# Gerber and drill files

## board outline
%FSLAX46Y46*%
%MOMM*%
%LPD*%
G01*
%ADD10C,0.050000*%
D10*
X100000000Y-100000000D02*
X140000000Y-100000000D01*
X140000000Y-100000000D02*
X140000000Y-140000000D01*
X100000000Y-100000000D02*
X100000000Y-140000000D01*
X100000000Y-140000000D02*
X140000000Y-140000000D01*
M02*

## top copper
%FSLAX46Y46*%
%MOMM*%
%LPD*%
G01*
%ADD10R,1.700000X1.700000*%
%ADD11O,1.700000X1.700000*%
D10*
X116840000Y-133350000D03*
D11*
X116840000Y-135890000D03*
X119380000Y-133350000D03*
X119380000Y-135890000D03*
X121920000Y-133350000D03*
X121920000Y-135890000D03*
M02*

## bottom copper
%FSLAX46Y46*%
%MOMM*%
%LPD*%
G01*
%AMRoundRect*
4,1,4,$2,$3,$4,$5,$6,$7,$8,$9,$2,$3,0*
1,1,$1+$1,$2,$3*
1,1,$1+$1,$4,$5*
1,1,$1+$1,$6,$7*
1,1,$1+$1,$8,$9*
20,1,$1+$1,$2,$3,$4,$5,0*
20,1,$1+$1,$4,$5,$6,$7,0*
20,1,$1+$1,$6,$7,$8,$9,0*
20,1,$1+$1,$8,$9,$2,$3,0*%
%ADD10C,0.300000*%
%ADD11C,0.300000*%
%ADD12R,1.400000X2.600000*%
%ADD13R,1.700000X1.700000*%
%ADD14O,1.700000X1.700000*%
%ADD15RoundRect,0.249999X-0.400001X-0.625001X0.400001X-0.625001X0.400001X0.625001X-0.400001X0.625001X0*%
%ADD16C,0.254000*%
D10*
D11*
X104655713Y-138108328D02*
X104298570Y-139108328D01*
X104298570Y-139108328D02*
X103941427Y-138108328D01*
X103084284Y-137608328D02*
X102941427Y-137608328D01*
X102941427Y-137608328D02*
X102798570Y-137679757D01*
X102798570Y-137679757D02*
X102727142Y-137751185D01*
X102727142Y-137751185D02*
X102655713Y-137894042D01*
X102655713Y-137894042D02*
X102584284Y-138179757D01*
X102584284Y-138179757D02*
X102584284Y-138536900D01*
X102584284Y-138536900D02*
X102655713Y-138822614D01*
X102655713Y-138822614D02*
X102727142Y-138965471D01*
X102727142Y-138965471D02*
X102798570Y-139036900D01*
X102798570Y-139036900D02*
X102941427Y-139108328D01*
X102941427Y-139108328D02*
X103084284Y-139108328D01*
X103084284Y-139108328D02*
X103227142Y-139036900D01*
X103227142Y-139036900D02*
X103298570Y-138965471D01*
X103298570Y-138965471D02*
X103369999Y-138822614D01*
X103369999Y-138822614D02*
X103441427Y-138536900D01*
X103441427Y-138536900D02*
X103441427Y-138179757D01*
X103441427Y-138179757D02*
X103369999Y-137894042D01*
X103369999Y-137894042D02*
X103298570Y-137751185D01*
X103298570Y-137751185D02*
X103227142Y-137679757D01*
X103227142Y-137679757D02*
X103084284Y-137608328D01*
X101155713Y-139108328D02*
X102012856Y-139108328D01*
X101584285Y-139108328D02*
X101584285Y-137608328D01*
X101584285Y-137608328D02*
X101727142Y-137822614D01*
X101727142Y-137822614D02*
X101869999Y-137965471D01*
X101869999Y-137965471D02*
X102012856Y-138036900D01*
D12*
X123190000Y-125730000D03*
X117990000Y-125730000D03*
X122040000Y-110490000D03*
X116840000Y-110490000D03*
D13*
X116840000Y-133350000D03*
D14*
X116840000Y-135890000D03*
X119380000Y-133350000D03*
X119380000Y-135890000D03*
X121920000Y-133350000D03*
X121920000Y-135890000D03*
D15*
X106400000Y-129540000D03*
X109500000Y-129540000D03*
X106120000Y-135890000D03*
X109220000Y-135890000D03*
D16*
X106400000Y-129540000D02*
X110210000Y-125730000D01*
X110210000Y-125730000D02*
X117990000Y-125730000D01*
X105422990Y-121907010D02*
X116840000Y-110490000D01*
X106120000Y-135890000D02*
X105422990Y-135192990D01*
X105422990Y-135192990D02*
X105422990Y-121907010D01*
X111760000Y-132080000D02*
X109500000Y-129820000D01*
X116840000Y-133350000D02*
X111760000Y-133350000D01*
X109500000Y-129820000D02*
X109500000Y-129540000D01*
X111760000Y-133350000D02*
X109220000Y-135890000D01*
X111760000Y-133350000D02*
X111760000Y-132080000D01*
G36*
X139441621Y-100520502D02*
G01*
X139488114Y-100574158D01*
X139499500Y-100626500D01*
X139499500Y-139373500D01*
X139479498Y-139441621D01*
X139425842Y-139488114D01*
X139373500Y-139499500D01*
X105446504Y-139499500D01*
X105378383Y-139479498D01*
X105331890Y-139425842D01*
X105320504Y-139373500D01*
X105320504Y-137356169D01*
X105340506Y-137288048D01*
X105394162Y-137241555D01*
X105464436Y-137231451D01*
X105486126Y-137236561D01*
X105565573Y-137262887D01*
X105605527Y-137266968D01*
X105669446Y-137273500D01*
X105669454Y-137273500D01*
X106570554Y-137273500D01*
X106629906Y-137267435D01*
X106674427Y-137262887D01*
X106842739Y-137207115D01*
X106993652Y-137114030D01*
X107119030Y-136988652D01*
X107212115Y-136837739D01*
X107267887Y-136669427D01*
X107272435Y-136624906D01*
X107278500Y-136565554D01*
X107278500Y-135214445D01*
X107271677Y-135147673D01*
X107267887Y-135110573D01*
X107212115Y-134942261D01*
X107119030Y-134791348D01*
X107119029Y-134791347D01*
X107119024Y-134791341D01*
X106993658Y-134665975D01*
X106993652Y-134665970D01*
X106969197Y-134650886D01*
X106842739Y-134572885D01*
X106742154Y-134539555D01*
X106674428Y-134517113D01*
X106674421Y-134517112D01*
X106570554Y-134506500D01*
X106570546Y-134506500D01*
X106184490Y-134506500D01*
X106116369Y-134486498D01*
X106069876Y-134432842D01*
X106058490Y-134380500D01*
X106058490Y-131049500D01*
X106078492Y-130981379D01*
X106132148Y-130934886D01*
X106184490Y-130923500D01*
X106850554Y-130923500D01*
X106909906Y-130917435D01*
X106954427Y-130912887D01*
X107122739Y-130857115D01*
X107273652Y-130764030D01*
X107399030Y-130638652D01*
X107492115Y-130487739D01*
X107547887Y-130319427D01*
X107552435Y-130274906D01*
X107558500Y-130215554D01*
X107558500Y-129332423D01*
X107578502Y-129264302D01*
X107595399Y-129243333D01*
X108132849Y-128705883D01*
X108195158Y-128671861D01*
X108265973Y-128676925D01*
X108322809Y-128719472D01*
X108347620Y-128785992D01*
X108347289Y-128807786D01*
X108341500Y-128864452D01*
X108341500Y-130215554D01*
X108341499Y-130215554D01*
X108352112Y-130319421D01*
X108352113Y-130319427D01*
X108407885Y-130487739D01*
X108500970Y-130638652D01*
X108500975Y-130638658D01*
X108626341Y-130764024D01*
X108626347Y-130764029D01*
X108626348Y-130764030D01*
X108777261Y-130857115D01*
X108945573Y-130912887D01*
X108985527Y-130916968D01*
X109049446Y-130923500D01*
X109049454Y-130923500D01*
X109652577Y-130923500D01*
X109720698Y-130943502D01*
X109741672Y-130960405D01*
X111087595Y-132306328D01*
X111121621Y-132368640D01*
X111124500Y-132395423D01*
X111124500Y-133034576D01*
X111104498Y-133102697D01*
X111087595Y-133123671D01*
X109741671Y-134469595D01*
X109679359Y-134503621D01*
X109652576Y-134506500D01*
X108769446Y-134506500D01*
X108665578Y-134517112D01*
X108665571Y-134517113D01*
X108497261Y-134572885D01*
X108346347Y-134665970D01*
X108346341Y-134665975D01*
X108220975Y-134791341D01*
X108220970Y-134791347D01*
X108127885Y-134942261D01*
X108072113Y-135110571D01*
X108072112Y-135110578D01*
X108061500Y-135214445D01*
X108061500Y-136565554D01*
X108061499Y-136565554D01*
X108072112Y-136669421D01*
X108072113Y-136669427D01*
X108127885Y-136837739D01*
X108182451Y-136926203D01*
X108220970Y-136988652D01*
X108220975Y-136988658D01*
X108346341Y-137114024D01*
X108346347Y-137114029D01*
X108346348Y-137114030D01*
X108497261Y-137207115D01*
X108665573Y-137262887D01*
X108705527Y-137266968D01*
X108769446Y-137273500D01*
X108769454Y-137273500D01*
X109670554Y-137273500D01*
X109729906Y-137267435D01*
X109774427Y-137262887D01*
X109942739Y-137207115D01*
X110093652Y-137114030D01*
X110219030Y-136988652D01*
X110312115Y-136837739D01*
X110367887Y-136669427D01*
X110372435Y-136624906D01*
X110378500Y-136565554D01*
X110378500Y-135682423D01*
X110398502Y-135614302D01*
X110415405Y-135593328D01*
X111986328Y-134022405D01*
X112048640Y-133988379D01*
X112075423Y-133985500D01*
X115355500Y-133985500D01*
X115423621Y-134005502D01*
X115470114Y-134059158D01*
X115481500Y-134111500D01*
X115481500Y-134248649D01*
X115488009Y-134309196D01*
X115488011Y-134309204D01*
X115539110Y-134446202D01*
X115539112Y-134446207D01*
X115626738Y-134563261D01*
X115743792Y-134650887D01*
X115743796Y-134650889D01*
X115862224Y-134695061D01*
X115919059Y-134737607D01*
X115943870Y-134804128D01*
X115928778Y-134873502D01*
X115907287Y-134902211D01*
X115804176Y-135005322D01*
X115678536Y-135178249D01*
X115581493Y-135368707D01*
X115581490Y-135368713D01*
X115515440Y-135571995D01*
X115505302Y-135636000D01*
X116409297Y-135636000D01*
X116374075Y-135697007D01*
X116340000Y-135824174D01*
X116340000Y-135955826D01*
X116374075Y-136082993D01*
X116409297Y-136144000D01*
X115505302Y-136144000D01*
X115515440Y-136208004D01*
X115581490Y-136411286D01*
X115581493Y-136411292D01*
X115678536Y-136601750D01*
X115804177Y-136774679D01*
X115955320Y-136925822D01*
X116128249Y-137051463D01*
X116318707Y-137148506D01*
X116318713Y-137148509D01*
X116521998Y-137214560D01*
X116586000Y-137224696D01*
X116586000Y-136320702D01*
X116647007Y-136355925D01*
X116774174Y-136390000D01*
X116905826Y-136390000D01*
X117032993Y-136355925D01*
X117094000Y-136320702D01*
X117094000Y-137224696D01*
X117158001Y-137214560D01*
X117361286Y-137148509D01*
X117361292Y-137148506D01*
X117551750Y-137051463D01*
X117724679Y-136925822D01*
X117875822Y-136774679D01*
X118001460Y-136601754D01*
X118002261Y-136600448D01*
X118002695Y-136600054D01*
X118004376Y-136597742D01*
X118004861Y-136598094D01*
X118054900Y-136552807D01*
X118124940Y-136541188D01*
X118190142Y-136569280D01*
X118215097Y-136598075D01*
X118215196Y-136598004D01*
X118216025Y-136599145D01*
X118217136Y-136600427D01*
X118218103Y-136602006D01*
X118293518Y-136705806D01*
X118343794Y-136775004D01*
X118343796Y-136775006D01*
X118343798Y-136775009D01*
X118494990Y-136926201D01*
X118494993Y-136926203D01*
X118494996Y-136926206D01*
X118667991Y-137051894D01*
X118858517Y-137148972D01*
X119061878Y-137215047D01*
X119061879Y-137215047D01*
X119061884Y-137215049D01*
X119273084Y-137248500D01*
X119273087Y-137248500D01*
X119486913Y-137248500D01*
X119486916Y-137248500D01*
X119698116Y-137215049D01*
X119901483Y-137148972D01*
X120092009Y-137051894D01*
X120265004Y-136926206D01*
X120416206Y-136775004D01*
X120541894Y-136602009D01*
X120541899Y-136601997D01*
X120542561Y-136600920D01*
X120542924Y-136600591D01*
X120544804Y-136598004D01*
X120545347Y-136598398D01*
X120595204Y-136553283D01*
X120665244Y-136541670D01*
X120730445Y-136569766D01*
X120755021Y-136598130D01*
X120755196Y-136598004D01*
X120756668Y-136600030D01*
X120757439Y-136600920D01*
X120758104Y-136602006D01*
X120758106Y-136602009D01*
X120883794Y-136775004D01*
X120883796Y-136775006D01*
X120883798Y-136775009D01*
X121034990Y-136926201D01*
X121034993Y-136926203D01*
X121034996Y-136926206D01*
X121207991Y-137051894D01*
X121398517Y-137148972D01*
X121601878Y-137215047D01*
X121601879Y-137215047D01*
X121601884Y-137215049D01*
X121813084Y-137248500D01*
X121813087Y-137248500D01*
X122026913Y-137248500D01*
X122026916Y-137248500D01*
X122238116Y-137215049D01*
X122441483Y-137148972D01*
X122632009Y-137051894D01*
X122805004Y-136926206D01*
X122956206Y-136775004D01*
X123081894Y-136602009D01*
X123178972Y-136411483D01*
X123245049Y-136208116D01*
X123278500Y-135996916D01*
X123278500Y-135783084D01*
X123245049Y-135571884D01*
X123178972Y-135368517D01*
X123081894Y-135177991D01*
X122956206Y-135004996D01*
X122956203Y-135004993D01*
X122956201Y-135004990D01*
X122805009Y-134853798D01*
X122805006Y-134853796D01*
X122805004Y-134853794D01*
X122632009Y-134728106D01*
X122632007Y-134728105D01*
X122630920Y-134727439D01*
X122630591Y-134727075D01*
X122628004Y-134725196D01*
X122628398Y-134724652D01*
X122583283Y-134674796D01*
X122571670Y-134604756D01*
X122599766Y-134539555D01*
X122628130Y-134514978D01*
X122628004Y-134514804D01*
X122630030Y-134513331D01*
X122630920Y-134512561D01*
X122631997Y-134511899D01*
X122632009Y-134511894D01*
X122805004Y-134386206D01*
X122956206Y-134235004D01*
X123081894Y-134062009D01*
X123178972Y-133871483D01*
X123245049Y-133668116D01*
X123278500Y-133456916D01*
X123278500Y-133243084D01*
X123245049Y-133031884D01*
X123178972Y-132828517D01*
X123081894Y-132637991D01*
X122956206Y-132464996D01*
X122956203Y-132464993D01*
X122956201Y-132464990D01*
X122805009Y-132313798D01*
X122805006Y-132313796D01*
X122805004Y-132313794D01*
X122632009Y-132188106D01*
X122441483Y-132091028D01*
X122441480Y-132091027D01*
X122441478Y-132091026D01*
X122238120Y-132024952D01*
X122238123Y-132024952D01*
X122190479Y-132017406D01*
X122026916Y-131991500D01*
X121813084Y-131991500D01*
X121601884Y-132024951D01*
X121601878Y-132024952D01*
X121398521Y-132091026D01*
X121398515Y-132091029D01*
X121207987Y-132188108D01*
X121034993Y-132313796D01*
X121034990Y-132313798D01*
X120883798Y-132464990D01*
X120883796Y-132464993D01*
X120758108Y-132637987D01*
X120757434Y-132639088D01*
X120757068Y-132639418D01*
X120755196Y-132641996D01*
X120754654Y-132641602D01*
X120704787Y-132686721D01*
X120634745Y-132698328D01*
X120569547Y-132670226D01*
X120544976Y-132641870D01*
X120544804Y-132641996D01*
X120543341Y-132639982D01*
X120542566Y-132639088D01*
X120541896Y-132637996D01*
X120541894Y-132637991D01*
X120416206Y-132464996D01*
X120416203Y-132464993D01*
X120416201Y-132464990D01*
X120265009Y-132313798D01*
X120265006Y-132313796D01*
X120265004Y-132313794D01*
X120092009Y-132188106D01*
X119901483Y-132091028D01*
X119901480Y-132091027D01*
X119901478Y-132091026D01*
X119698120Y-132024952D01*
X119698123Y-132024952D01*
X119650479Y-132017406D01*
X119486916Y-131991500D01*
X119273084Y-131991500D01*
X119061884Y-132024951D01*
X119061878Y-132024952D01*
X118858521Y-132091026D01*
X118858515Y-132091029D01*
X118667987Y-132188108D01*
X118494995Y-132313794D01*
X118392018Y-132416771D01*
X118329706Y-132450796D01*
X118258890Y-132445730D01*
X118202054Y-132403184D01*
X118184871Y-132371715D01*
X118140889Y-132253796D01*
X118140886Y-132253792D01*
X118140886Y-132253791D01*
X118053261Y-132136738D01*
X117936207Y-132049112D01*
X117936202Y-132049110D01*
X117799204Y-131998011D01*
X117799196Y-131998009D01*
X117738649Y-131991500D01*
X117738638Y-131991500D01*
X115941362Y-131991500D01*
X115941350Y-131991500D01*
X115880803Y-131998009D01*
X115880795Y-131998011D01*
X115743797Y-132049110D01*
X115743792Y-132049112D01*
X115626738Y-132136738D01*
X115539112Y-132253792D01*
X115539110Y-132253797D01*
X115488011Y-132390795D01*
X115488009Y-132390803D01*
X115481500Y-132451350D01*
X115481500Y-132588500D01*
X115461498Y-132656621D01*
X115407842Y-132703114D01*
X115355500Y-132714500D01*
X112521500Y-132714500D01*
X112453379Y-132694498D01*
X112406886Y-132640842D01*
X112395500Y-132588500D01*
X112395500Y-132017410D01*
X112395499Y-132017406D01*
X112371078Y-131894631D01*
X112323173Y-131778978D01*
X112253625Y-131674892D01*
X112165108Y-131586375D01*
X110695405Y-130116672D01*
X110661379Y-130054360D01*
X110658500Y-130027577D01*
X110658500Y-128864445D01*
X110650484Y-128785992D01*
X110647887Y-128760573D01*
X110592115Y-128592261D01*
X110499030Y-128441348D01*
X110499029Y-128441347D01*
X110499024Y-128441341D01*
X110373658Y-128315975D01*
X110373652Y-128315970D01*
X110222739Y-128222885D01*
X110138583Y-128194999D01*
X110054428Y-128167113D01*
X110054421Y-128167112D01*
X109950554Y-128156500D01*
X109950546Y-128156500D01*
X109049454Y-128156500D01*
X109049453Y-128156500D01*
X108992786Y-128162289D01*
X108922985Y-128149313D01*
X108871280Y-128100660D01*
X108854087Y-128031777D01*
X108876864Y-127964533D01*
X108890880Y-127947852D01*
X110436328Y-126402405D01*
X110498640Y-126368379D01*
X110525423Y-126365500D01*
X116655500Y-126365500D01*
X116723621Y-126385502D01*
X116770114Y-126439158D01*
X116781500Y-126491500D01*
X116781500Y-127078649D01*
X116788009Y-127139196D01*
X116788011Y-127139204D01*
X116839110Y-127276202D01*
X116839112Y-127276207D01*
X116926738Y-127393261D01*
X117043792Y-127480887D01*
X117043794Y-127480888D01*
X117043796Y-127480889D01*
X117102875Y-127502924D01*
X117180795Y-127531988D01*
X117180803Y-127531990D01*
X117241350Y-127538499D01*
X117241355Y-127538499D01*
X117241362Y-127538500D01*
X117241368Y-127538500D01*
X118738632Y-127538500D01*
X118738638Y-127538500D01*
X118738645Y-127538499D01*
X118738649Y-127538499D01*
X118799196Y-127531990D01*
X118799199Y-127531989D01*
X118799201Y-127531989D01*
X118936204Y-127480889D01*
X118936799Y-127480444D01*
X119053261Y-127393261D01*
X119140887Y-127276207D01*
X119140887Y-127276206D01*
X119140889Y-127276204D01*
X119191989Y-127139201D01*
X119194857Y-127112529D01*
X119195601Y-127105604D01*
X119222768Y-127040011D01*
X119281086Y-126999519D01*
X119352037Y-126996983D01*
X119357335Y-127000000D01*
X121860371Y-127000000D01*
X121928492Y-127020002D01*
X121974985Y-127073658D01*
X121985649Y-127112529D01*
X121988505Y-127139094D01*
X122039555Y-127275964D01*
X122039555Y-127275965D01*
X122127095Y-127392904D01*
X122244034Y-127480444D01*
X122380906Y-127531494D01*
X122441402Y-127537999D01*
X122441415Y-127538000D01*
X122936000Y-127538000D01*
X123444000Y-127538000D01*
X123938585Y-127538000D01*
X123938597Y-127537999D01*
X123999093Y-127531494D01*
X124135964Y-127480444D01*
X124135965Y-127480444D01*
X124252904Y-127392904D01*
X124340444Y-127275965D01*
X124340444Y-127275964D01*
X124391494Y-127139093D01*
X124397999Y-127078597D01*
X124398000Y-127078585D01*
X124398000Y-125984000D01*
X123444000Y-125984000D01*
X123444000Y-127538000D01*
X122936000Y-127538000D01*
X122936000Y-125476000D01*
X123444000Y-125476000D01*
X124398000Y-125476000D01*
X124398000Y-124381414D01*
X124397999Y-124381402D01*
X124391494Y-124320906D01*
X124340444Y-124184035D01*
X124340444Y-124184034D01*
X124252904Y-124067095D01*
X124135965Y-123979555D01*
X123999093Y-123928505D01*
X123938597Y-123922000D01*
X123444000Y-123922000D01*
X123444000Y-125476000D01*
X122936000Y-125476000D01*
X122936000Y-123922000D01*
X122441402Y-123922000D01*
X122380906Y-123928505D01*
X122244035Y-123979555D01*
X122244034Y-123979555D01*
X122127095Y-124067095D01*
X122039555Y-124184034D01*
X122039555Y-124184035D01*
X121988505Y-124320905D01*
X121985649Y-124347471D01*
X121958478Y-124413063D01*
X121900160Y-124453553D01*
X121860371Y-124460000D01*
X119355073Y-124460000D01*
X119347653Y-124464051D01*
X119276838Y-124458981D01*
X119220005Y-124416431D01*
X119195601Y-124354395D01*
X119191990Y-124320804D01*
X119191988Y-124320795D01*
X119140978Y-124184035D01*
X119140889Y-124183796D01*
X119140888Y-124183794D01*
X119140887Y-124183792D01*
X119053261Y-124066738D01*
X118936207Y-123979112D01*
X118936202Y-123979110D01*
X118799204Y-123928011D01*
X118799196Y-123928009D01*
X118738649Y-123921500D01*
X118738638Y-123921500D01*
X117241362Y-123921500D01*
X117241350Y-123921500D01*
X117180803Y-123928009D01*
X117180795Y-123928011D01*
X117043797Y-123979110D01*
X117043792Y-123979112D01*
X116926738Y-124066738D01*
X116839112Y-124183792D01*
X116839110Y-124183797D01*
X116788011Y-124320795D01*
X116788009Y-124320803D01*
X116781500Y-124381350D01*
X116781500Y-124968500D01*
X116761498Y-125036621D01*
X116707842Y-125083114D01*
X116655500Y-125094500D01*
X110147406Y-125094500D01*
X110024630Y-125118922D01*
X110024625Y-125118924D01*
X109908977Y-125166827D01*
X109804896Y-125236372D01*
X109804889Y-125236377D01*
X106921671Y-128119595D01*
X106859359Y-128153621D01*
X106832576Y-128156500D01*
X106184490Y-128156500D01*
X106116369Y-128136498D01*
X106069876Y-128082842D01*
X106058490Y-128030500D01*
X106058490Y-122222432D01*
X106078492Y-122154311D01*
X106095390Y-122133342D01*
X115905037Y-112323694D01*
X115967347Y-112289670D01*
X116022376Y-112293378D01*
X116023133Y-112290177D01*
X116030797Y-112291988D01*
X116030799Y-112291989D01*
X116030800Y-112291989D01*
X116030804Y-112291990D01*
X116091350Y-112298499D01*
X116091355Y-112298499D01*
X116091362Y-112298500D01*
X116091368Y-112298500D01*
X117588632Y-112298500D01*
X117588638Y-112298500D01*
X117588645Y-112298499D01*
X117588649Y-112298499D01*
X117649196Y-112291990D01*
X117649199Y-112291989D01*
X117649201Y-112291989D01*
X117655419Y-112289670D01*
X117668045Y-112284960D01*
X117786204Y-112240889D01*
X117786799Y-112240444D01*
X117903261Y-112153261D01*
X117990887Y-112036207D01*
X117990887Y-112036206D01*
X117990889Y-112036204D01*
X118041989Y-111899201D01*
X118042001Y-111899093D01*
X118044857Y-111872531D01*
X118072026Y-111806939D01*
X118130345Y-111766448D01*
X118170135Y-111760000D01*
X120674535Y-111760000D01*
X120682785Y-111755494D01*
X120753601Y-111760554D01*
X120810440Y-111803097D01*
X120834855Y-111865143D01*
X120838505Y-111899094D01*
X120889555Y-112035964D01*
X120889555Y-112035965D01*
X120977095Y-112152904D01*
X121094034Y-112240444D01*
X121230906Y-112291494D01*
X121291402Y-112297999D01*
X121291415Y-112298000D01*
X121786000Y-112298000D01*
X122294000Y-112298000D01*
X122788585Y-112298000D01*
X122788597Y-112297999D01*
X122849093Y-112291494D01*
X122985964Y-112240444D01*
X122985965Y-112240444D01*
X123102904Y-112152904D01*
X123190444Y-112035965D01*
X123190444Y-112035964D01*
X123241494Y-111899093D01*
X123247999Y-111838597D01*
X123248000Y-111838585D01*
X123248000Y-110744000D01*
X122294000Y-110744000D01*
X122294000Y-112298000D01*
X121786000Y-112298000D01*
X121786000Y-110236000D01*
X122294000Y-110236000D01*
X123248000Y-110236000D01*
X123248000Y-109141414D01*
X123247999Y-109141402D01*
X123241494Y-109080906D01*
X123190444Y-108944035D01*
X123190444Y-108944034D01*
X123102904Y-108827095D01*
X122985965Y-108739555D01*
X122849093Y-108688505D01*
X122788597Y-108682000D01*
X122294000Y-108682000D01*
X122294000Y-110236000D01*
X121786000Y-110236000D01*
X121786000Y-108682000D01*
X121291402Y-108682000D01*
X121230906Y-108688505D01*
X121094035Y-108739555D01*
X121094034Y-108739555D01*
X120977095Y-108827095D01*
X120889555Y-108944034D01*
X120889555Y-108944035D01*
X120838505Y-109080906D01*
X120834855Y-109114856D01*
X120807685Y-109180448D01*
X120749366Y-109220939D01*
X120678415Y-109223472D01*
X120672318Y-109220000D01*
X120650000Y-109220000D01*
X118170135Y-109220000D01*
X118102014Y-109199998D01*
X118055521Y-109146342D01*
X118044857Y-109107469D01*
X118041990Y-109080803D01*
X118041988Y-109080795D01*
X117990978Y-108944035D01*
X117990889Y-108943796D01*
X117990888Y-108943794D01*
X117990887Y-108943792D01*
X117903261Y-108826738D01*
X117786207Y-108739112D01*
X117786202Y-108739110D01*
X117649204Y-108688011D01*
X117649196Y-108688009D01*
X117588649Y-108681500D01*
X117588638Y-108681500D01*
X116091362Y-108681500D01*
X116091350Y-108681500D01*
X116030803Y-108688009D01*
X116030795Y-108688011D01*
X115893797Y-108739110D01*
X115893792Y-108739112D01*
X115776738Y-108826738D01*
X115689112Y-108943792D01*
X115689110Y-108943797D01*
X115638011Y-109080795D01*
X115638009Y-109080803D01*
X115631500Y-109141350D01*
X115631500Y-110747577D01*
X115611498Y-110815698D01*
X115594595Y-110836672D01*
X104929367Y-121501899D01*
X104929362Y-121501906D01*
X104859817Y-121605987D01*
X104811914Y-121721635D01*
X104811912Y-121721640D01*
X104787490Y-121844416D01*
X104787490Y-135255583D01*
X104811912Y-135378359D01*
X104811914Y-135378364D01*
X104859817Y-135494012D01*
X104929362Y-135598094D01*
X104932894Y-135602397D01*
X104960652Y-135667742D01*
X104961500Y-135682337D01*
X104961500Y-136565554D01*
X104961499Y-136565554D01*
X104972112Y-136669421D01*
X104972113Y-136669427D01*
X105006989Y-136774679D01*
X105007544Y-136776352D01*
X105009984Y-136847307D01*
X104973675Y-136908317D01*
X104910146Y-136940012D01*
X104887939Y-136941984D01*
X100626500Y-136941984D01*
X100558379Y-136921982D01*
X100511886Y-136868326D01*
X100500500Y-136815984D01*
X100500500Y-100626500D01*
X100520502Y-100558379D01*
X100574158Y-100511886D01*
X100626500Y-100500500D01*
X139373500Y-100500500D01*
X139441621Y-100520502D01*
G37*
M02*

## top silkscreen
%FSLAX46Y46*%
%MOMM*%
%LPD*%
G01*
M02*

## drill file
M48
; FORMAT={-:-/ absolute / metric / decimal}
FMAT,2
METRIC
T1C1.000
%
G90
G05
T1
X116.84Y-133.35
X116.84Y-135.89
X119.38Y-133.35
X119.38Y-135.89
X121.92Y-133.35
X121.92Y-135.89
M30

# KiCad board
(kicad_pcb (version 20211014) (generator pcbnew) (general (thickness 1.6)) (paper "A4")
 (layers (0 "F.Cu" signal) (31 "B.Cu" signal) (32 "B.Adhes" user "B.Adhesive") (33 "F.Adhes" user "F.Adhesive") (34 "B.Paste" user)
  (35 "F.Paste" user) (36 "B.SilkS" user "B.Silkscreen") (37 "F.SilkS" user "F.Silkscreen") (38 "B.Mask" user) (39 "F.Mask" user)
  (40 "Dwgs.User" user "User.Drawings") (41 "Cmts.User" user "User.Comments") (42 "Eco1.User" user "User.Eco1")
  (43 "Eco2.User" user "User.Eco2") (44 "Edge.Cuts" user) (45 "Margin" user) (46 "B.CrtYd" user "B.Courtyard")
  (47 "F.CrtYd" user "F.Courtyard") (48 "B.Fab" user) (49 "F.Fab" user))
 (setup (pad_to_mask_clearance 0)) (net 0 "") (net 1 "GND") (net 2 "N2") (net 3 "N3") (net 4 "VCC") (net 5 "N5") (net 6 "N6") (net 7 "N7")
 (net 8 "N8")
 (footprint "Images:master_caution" (layer "F.Cu") (at 119.038703 118.605147)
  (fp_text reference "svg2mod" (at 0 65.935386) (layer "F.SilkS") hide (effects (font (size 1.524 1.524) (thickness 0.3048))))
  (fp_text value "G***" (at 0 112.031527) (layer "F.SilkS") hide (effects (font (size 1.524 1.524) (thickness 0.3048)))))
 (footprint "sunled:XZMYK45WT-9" (layer "B.Cu") (at 120.59 125.73 180)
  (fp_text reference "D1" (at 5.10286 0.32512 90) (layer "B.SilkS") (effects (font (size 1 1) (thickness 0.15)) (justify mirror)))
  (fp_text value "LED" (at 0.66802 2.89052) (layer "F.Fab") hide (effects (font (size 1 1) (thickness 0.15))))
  (pad "1" smd rect locked (at -2.6 0 180) (size 1.4 2.6) (layers "B.Cu" "B.Paste" "B.Mask") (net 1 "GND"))
  (pad "2" smd rect locked (at 2.6 0 180) (size 1.4 2.6) (layers "B.Cu" "B.Paste" "B.Mask") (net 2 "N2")))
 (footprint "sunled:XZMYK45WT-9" (layer "B.Cu") (at 119.44 110.49 180)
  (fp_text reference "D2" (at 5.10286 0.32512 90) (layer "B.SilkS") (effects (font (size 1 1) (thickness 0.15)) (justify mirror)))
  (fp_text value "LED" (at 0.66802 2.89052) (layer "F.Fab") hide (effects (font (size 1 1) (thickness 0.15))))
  (pad "1" smd rect locked (at -2.6 0 180) (size 1.4 2.6) (layers "B.Cu" "B.Paste" "B.Mask") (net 1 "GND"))
  (pad "2" smd rect locked (at 2.6 0 180) (size 1.4 2.6) (layers "B.Cu" "B.Paste" "B.Mask") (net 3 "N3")))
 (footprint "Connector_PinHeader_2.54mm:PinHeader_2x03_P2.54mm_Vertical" (layer "B.Cu") (at 116.84 133.35 -90)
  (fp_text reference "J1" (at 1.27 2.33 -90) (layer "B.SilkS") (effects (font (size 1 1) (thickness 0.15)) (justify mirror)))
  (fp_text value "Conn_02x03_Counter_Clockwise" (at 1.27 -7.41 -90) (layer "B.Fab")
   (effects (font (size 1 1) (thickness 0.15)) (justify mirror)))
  (pad "1" thru_hole rect locked (at 0 0 270) (size 1.7 1.7) (drill 1) (layers *.Cu *.Mask) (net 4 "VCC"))
  (pad "2" thru_hole oval locked (at 2.54 0 270) (size 1.7 1.7) (drill 1) (layers *.Cu *.Mask) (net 1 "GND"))
  (pad "3" thru_hole oval locked (at 0 -2.54 270) (size 1.7 1.7) (drill 1) (layers *.Cu *.Mask) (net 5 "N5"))
  (pad "4" thru_hole oval locked (at 2.54 -2.54 270) (size 1.7 1.7) (drill 1) (layers *.Cu *.Mask) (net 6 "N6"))
  (pad "5" thru_hole oval locked (at 0 -5.08 270) (size 1.7 1.7) (drill 1) (layers *.Cu *.Mask) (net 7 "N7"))
  (pad "6" thru_hole oval locked (at 2.54 -5.08 270) (size 1.7 1.7) (drill 1) (layers *.Cu *.Mask) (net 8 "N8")))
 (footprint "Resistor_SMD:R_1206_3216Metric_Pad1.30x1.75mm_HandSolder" (layer "B.Cu") (at 107.95 129.54)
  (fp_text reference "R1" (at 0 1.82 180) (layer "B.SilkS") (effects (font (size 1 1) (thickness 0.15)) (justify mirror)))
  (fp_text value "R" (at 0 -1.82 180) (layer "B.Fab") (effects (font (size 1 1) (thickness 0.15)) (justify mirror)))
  (pad "1" smd roundrect locked (at -1.55 0) (size 1.3 1.75) (layers "B.Cu" "B.Paste" "B.Mask") (roundrect_rratio 0.1923069231) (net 2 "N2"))
  (pad "2" smd roundrect locked (at 1.55 0) (size 1.3 1.75) (layers "B.Cu" "B.Paste" "B.Mask") (roundrect_rratio 0.1923069231) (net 4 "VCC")))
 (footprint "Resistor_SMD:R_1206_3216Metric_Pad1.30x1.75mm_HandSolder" (layer "B.Cu") (at 107.67 135.89)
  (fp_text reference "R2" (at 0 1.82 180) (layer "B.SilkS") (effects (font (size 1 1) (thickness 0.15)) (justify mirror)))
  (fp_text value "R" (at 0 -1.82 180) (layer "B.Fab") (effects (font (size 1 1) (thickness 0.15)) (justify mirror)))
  (pad "1" smd roundrect locked (at -1.55 0) (size 1.3 1.75) (layers "B.Cu" "B.Paste" "B.Mask") (roundrect_rratio 0.1923069231) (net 3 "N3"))
  (pad "2" smd roundrect locked (at 1.55 0) (size 1.3 1.75) (layers "B.Cu" "B.Paste" "B.Mask") (roundrect_rratio 0.1923069231) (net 4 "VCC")))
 (gr_line (start 100 100) (end 140 100) (layer "Edge.Cuts") (width 0.05))
 (gr_line (start 140 100) (end 140 140) (layer "Edge.Cuts") (width 0.05))
 (gr_line (start 100 100) (end 100 140) (layer "Edge.Cuts") (width 0.05))
 (gr_line (start 100 140) (end 140 140) (layer "Edge.Cuts") (width 0.05))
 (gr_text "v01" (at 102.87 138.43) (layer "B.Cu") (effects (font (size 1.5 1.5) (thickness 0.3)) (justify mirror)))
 (segment (start 106.4 129.54) (end 110.21 125.73) (width 0.254) (layer "B.Cu") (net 2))
 (segment (start 110.21 125.73) (end 117.99 125.73) (width 0.254) (layer "B.Cu") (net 2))
 (segment (start 105.42299 121.90701) (end 116.84 110.49) (width 0.254) (layer "B.Cu") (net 3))
 (segment (start 106.12 135.89) (end 105.42299 135.19299) (width 0.254) (layer "B.Cu") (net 3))
 (segment (start 105.42299 135.19299) (end 105.42299 121.90701) (width 0.254) (layer "B.Cu") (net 3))
 (segment (start 111.76 132.08) (end 109.5 129.82) (width 0.254) (layer "B.Cu") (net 4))
 (segment (start 116.84 133.35) (end 111.76 133.35) (width 0.254) (layer "B.Cu") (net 4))
 (segment (start 109.5 129.82) (end 109.5 129.54) (width 0.254) (layer "B.Cu") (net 4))
 (segment (start 111.76 133.35) (end 109.22 135.89) (width 0.254) (layer "B.Cu") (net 4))
 (segment (start 111.76 133.35) (end 111.76 132.08) (width 0.254) (layer "B.Cu") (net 4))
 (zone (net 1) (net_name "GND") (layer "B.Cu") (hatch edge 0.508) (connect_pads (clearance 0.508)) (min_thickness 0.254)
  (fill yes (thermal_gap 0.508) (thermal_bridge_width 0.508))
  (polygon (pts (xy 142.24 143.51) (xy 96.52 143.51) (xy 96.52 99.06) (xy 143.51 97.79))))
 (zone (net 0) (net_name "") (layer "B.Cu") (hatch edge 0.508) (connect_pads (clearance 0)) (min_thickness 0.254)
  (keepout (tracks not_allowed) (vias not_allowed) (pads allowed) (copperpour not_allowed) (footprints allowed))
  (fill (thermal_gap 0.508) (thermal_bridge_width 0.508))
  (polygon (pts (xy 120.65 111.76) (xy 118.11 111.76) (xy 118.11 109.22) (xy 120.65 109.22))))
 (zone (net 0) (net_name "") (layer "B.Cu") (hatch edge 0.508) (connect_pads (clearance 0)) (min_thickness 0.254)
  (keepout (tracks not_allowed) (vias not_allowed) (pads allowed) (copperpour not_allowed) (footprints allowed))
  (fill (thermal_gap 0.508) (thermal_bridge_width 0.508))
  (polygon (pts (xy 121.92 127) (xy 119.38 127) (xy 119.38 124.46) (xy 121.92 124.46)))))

